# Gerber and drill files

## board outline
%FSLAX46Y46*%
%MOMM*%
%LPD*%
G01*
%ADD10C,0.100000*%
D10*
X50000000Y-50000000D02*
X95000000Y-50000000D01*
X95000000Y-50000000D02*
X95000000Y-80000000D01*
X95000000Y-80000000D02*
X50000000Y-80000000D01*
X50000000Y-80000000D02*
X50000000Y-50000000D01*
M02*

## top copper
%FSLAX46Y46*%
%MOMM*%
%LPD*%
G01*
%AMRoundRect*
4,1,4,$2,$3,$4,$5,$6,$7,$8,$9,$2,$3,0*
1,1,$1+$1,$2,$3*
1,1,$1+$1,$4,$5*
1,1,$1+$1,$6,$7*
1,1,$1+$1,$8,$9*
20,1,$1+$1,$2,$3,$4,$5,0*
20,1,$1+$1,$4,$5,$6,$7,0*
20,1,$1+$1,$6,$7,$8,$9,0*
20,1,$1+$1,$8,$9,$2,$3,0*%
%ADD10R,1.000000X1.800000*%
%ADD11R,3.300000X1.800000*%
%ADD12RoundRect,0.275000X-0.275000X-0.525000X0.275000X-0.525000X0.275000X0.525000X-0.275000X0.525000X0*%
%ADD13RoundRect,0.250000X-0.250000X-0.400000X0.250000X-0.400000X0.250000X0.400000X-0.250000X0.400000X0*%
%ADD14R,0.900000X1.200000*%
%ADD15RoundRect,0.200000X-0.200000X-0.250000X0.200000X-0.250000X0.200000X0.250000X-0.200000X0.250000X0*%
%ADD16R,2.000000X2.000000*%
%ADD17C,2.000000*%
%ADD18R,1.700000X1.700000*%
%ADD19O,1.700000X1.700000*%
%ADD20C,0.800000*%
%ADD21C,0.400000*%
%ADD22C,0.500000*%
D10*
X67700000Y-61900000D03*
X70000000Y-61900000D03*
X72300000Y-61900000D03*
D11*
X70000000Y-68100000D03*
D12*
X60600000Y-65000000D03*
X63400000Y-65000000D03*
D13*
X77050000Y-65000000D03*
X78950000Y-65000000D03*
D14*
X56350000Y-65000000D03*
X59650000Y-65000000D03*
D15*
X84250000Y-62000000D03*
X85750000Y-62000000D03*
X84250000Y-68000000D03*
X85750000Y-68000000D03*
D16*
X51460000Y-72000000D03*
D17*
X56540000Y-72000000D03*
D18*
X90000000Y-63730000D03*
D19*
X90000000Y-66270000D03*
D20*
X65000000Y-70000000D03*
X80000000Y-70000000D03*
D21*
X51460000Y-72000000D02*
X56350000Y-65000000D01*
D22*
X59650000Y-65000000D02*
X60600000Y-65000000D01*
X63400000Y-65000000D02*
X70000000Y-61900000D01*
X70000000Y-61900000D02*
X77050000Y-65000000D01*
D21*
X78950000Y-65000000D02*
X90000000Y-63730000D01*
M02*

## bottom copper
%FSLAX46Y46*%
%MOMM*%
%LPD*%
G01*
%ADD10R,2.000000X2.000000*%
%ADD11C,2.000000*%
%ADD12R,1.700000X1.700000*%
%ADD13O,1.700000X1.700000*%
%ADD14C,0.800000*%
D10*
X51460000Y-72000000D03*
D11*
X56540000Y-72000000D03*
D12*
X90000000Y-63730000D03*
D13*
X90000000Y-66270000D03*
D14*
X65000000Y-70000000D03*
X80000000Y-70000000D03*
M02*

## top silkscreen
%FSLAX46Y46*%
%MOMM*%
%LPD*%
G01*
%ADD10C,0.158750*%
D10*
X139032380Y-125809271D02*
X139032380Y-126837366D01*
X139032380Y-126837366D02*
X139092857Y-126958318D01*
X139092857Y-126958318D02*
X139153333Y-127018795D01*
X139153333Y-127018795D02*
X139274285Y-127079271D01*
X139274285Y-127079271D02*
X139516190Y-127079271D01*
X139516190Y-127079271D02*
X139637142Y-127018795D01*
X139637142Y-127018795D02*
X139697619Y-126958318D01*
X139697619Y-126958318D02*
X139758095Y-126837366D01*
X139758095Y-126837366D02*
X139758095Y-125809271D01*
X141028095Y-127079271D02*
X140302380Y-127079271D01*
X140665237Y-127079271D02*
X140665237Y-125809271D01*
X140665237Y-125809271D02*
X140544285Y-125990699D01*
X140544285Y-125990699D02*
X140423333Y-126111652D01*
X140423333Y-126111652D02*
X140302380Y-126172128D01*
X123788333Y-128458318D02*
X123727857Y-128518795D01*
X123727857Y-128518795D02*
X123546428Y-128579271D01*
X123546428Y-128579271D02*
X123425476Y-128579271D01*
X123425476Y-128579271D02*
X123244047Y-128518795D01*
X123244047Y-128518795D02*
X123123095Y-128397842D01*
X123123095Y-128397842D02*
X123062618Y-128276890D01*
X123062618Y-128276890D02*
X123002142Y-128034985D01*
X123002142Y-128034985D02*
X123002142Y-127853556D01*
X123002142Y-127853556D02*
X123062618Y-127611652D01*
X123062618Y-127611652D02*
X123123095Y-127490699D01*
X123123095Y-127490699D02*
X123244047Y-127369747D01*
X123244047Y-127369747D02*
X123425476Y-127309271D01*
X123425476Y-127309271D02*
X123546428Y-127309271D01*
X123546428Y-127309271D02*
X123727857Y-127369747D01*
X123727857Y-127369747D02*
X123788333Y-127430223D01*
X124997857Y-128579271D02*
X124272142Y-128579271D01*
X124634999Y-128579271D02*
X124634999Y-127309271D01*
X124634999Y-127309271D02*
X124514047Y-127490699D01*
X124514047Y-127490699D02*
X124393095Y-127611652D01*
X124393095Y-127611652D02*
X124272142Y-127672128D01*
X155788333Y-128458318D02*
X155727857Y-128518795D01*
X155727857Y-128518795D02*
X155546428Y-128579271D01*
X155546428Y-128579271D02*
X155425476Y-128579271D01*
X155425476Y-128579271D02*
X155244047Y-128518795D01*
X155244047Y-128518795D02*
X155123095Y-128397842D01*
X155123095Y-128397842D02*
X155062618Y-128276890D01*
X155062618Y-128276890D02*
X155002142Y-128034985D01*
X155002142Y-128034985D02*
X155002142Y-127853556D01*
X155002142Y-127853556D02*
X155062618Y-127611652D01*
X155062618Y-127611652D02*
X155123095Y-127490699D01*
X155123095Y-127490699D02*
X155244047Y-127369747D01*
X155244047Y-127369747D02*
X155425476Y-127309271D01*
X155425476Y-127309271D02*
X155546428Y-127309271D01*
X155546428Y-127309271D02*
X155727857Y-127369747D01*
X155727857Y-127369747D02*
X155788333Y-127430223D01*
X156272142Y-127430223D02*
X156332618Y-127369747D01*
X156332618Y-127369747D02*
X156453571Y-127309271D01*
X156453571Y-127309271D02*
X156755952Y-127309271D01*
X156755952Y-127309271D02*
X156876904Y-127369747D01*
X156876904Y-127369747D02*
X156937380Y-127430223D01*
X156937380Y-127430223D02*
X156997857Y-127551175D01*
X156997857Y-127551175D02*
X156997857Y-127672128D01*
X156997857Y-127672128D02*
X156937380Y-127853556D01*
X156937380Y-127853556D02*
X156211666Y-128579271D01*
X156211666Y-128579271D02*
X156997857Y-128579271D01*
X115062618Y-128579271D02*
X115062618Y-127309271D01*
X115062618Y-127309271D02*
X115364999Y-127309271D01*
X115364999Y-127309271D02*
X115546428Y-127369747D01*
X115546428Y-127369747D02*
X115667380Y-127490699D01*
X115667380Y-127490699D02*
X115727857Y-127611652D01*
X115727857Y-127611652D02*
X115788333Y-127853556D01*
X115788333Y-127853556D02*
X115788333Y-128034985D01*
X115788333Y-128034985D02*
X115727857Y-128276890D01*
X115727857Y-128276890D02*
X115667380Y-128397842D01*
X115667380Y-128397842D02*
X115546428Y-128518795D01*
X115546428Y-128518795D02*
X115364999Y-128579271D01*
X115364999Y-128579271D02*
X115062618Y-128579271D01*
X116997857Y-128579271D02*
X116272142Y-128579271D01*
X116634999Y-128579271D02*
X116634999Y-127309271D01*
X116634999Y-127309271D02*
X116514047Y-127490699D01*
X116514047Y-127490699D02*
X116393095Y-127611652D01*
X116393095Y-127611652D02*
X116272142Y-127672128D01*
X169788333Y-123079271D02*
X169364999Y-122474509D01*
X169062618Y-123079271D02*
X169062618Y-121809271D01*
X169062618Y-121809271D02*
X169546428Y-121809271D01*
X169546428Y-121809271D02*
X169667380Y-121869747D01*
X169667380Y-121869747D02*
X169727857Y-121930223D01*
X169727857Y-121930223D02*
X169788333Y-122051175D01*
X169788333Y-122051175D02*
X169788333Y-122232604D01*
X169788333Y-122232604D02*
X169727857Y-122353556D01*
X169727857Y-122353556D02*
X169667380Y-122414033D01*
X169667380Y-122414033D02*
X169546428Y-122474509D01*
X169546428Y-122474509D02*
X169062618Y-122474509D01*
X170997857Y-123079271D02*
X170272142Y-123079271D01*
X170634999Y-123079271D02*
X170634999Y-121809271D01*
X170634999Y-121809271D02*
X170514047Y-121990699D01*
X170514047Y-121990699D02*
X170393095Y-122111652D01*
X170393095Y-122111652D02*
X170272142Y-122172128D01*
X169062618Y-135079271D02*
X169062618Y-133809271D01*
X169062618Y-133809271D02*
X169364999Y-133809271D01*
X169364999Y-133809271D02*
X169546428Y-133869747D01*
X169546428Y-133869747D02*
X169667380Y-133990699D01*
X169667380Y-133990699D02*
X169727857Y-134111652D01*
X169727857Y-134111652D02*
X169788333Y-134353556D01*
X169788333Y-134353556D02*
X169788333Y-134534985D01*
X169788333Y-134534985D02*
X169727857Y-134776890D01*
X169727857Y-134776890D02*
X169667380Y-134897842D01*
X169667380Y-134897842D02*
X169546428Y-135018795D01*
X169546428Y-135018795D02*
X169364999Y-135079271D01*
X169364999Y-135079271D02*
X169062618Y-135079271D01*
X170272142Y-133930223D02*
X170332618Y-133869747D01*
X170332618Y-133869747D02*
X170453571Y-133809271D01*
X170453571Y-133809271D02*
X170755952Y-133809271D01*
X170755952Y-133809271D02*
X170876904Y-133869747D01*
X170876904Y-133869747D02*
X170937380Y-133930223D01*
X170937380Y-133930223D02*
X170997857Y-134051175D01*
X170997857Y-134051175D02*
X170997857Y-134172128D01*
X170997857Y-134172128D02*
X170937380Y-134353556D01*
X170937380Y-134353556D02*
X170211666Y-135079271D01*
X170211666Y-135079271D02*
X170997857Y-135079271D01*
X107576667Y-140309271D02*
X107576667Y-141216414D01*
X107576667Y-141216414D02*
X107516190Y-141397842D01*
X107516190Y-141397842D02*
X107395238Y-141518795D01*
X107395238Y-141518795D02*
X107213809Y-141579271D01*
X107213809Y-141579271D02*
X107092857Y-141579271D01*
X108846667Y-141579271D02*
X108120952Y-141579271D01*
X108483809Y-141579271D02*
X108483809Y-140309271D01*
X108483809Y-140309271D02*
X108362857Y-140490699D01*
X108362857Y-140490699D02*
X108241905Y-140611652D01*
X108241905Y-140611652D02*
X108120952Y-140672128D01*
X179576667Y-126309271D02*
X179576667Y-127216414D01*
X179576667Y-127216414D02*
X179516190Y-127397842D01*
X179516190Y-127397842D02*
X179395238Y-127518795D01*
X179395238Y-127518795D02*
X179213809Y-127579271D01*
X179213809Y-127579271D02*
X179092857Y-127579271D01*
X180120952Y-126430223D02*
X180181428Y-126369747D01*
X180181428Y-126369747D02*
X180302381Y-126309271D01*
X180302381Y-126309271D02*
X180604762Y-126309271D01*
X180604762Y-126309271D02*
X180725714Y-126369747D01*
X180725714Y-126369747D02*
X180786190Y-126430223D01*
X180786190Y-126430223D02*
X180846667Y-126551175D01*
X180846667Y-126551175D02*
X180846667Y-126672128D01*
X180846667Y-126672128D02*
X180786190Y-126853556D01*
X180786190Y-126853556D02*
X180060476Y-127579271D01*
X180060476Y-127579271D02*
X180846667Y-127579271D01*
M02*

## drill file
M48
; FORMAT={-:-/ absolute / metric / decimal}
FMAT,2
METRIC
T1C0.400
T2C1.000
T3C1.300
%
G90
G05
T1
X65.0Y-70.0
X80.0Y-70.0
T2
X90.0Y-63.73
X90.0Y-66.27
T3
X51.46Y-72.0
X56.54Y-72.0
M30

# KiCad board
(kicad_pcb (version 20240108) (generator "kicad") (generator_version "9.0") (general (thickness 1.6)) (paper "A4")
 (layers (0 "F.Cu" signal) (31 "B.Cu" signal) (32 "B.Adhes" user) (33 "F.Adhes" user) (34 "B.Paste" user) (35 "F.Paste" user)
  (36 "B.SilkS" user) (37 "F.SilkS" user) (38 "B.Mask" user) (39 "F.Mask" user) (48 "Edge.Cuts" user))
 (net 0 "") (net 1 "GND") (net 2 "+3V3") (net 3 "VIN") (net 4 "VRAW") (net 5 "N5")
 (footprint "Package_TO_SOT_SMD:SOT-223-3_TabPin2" (layer "F.Cu") (at 70.0 65.0) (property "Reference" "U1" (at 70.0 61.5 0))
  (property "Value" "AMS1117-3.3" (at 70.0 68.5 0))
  (pad "1" smd rect (at -2.3 -3.1) (size 1.0 1.8) (layers "F.Cu" "F.Mask") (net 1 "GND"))
  (pad "2" smd rect (at 0.0 -3.1) (size 1.0 1.8) (layers "F.Cu" "F.Mask") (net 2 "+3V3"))
  (pad "3" smd rect (at 2.3 -3.1) (size 1.0 1.8) (layers "F.Cu" "F.Mask") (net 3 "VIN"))
  (pad "4" smd rect (at 0.0 3.1) (size 3.3 1.8) (layers "F.Cu" "F.Mask") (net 2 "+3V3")))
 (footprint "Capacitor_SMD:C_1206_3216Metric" (layer "F.Cu") (at 62.0 65.0) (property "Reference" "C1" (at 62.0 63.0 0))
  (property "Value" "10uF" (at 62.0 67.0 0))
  (pad "1" smd roundrect (at -1.4 0) (size 1.1 1.6) (layers "F.Cu" "F.Mask") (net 3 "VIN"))
  (pad "2" smd roundrect (at 1.4 0) (size 1.1 1.6) (layers "F.Cu" "F.Mask") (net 1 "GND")))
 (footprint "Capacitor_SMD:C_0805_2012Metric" (layer "F.Cu") (at 78.0 65.0) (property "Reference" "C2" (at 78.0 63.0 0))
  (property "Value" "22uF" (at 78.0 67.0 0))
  (pad "1" smd roundrect (at -0.95 0) (size 1.0 1.3) (layers "F.Cu" "F.Mask") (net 2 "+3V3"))
  (pad "2" smd roundrect (at 0.95 0) (size 1.0 1.3) (layers "F.Cu" "F.Mask") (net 1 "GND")))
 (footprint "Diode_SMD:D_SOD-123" (layer "F.Cu") (at 58.0 65.0) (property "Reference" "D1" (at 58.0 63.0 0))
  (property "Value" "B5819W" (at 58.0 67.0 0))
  (pad "1" smd rect (at -1.65 0) (size 0.9 1.2) (layers "F.Cu" "F.Mask") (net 3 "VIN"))
  (pad "2" smd rect (at 1.65 0) (size 0.9 1.2) (layers "F.Cu" "F.Mask") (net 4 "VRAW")))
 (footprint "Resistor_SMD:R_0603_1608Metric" (layer "F.Cu") (at 85.0 62.0) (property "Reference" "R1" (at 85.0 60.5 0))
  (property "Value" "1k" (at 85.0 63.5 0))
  (pad "1" smd roundrect (at -0.75 0) (size 0.8 0.9) (layers "F.Cu" "F.Mask") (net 2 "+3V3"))
  (pad "2" smd roundrect (at 0.75 0) (size 0.8 0.9) (layers "F.Cu" "F.Mask") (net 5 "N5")))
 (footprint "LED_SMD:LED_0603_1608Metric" (layer "F.Cu") (at 85.0 68.0) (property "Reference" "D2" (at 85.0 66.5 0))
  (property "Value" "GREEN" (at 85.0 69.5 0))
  (pad "1" smd roundrect (at -0.75 0) (size 0.8 0.9) (layers "F.Cu" "F.Mask") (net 1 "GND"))
  (pad "2" smd roundrect (at 0.75 0) (size 0.8 0.9) (layers "F.Cu" "F.Mask") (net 5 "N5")))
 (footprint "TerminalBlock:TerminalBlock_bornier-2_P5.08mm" (layer "F.Cu") (at 54.0 72.0) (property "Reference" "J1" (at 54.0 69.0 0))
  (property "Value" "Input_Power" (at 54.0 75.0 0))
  (pad "1" thru_hole rect (at -2.54 0) (size 2.0 2.0) (drill 1.3) (layers "*.Cu" "*.Mask") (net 4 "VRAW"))
  (pad "2" thru_hole circle (at 2.54 0) (size 2.0 2.0) (drill 1.3) (layers "*.Cu" "*.Mask") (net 1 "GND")))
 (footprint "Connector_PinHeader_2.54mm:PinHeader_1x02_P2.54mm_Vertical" (layer "F.Cu") (at 90.0 65.0)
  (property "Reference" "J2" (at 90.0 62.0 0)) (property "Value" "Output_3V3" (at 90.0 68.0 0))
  (pad "1" thru_hole rect (at 0 -1.27) (size 1.7 1.7) (drill 1.0) (layers "*.Cu" "*.Mask") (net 2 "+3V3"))
  (pad "2" thru_hole oval (at 0 1.27) (size 1.7 1.7) (drill 1.0) (layers "*.Cu" "*.Mask") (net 1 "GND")))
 (segment (start 51.46 72.0) (end 56.35 65.0) (width 0.4) (layer "F.Cu") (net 4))
 (segment (start 59.65 65.0) (end 60.6 65.0) (width 0.5) (layer "F.Cu") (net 3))
 (segment (start 63.4 65.0) (end 70.0 61.9) (width 0.5) (layer "F.Cu") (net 3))
 (segment (start 70.0 61.9) (end 77.05 65.0) (width 0.5) (layer "F.Cu") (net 2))
 (segment (start 78.95 65.0) (end 90.0 63.73) (width 0.4) (layer "F.Cu") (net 2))
 (via (at 65.0 70.0) (size 0.8) (drill 0.4) (layers "F.Cu" "B.Cu") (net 1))
 (via (at 80.0 70.0) (size 0.8) (drill 0.4) (layers "F.Cu" "B.Cu") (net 1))
 (gr_line (start 50.0 50.0) (end 95.0 50.0) (layer "Edge.Cuts") (width 0.1))
 (gr_line (start 95.0 50.0) (end 95.0 80.0) (layer "Edge.Cuts") (width 0.1))
 (gr_line (start 95.0 80.0) (end 50.0 80.0) (layer "Edge.Cuts") (width 0.1))
 (gr_line (start 50.0 80.0) (end 50.0 50.0) (layer "Edge.Cuts") (width 0.1)))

